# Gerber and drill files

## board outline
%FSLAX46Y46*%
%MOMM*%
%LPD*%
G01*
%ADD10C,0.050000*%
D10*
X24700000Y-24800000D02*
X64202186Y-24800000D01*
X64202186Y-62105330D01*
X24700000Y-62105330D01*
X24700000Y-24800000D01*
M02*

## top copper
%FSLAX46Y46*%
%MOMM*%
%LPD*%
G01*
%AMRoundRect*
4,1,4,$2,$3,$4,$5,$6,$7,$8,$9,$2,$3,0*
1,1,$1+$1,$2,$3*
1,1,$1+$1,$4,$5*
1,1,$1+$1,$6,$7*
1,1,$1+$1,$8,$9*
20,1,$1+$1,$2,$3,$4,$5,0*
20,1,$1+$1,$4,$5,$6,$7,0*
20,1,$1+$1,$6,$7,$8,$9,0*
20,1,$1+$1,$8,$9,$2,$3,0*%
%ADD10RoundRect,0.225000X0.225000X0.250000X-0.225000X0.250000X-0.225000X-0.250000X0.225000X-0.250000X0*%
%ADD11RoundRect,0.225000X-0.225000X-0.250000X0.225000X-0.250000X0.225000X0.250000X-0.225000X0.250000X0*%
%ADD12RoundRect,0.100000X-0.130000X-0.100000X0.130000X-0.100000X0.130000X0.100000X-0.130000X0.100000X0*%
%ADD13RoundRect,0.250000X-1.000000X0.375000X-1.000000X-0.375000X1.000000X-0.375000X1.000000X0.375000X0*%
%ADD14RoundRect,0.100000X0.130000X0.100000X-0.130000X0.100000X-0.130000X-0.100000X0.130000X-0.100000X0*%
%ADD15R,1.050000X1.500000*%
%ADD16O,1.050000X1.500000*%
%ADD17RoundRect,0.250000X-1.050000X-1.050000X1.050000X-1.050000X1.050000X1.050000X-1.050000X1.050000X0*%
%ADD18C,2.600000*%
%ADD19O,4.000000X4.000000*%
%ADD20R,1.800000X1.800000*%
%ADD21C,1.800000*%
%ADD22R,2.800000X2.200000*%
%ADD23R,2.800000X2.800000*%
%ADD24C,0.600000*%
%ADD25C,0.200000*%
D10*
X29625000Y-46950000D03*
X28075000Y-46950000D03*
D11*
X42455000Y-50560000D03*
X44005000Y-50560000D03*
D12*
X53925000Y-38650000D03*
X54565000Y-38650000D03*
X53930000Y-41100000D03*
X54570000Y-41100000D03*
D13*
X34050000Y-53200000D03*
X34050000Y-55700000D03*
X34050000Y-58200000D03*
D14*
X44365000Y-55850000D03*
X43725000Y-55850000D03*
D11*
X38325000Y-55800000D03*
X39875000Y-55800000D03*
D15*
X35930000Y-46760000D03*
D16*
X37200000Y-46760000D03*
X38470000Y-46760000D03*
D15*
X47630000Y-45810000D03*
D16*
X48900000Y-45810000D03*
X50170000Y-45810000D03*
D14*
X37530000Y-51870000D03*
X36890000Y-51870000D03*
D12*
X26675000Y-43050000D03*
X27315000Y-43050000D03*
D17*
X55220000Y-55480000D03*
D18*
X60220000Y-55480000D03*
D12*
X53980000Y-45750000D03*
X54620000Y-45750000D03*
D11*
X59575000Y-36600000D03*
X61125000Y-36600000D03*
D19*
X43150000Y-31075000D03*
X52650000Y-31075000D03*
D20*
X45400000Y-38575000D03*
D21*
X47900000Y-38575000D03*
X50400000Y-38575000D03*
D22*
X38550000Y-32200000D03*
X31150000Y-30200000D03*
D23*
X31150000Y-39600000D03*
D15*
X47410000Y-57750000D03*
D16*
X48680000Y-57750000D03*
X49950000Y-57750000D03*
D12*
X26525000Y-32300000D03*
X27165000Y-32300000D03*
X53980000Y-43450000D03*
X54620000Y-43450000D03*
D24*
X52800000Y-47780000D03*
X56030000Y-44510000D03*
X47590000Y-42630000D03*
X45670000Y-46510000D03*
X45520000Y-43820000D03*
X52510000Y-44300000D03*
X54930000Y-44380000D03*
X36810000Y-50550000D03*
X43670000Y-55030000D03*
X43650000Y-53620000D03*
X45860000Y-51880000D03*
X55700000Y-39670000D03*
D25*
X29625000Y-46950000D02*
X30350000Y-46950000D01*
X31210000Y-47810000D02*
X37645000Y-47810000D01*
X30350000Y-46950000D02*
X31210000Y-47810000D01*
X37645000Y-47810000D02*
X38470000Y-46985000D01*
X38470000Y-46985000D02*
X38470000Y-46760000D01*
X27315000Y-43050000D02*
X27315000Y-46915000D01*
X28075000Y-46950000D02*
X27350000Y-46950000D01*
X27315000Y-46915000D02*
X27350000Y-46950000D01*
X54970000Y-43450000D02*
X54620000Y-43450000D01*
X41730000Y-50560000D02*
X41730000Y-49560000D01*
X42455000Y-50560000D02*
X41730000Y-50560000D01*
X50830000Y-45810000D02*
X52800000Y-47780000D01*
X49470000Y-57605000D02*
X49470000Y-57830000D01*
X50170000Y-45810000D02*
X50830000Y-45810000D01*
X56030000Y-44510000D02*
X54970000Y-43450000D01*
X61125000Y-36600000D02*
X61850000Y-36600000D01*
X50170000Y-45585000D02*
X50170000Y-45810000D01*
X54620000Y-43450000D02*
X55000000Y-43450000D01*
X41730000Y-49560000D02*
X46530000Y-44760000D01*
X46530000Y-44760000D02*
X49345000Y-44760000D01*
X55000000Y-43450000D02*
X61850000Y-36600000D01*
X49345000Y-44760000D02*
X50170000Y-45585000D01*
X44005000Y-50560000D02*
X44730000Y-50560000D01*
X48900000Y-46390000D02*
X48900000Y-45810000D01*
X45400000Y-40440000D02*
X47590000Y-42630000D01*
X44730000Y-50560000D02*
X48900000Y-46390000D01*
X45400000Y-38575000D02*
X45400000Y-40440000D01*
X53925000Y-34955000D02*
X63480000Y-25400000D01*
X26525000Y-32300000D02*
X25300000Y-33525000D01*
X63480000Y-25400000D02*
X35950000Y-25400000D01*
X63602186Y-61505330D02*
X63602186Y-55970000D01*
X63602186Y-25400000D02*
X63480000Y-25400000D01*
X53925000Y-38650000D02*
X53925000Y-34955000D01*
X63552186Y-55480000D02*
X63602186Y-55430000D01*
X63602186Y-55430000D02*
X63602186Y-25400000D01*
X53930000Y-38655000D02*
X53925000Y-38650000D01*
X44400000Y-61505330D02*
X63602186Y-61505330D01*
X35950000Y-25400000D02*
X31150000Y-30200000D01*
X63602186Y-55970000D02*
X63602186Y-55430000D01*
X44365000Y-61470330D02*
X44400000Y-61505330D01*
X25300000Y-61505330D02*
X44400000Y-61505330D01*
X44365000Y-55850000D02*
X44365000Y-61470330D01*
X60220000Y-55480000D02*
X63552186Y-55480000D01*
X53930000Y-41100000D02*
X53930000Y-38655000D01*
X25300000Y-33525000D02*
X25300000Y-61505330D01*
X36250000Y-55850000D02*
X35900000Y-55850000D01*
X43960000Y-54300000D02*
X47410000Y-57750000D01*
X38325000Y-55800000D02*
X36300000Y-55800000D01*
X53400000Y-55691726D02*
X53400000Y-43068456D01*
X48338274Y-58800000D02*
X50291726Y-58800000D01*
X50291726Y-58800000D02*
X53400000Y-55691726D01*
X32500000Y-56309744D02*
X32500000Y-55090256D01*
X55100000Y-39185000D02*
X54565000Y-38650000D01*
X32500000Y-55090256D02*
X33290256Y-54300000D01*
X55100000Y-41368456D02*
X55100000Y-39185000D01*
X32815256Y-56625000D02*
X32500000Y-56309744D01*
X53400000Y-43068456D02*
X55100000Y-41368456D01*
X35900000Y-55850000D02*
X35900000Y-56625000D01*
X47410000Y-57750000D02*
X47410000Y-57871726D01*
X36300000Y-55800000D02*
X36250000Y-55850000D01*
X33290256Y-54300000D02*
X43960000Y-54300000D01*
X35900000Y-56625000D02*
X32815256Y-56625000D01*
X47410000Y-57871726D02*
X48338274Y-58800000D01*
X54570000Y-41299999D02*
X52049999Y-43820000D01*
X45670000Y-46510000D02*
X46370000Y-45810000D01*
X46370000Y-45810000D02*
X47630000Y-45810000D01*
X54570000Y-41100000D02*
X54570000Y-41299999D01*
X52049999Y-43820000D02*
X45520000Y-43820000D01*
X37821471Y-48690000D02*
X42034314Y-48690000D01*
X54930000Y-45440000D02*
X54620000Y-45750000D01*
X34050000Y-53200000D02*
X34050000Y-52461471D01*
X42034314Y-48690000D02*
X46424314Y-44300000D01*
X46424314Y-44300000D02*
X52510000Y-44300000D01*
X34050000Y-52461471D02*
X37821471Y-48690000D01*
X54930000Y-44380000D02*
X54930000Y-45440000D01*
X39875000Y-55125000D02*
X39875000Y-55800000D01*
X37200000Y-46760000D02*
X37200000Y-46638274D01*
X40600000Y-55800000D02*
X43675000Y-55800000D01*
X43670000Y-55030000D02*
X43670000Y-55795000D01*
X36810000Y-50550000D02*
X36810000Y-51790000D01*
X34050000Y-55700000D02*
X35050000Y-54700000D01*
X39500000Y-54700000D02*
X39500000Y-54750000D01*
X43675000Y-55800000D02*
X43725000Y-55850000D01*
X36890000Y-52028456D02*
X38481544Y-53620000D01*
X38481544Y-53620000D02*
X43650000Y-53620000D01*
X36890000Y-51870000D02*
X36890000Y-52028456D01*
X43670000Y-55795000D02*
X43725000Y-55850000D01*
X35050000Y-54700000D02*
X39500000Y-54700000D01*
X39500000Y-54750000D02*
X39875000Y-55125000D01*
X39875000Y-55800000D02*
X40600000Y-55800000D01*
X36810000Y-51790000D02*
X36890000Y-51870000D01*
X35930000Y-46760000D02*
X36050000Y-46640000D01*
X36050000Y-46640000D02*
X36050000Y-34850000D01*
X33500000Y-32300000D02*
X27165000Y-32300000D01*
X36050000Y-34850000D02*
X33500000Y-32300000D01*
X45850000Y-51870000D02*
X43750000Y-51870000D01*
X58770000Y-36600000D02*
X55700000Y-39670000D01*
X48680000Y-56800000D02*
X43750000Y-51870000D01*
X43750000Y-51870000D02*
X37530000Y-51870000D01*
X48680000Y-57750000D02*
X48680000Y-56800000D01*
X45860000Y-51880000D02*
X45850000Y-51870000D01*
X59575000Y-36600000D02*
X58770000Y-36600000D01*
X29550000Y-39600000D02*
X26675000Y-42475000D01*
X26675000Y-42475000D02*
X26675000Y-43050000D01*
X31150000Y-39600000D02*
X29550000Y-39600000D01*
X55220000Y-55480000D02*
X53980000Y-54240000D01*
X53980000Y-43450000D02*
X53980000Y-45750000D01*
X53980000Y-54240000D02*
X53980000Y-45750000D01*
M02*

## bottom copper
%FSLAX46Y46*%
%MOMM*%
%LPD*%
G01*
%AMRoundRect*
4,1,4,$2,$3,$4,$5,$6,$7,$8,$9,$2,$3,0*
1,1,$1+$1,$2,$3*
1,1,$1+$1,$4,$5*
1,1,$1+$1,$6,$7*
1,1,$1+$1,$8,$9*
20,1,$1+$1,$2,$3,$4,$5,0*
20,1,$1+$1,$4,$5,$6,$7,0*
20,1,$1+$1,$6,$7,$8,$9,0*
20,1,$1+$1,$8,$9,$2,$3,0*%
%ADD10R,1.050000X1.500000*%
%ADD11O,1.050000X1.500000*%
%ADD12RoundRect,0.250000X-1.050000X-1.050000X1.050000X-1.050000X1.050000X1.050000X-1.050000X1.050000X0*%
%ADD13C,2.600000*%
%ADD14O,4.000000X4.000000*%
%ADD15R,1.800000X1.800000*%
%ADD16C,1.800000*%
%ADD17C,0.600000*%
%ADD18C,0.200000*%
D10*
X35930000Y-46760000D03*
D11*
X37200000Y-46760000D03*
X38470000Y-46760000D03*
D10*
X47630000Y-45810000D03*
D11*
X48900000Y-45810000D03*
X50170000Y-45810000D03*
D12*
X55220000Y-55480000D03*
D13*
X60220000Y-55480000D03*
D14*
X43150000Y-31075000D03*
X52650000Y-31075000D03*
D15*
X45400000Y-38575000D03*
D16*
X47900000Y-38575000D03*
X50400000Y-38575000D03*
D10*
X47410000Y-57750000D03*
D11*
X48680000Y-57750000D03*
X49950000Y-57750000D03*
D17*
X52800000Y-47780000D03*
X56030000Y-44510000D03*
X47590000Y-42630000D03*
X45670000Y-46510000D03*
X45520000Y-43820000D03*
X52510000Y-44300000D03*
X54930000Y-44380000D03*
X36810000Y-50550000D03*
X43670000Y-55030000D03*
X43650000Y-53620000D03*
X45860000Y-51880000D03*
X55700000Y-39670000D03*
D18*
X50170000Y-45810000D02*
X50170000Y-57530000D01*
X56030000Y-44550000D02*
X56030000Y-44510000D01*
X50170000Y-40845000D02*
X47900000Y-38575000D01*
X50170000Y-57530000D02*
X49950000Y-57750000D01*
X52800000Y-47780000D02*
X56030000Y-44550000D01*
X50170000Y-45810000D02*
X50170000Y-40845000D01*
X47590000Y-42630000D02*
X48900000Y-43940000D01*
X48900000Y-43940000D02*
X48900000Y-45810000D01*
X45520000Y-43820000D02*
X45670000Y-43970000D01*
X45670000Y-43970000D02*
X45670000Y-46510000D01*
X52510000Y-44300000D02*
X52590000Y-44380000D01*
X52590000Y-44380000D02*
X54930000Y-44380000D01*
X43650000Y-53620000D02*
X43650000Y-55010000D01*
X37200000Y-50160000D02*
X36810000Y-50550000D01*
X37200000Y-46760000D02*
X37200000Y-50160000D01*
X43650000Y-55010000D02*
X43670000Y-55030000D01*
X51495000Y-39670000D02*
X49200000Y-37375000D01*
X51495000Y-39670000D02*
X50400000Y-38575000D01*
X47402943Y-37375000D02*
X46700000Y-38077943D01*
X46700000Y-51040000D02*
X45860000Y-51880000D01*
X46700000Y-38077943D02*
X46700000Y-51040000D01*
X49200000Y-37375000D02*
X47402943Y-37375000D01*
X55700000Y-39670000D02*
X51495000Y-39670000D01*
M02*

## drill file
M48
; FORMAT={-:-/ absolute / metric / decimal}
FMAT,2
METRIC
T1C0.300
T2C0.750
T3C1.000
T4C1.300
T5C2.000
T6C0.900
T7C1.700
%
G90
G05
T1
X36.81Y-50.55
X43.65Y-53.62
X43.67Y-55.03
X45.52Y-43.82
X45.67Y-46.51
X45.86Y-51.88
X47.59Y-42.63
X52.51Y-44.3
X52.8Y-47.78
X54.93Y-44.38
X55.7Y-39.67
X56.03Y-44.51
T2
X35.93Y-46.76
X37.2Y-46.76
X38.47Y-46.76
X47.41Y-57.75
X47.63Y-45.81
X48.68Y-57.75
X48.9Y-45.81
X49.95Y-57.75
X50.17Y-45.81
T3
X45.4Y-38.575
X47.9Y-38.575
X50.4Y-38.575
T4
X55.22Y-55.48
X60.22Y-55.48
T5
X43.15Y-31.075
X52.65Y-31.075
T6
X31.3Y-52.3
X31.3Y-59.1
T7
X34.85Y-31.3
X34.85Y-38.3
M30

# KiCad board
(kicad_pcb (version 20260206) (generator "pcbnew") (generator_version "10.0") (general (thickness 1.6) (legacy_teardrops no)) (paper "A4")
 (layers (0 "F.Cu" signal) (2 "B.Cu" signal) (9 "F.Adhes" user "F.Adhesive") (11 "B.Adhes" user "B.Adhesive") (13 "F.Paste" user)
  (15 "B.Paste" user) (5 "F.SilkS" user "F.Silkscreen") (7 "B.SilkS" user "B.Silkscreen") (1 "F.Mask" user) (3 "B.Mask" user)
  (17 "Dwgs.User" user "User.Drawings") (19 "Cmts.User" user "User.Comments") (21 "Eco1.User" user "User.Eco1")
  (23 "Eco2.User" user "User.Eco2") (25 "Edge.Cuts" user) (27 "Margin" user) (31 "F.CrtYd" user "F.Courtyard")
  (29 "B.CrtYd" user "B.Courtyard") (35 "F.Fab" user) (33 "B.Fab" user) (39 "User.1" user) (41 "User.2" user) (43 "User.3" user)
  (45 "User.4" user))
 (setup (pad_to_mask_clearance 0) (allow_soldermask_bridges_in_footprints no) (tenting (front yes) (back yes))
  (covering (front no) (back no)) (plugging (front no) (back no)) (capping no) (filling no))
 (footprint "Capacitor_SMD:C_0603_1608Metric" (layer "F.Cu") (at 28.85 46.95 180)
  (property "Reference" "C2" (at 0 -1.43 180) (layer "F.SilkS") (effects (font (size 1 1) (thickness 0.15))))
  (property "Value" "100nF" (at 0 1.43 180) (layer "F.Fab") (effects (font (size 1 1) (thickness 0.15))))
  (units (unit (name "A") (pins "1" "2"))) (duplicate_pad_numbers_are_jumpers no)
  (pad "1" smd roundrect (at -0.775 0 180) (size 0.9 0.95) (layers "F.Cu" "F.Mask" "F.Paste") (roundrect_rratio 0.25) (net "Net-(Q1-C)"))
  (pad "2" smd roundrect (at 0.775 0 180) (size 0.9 0.95) (layers "F.Cu" "F.Mask" "F.Paste") (roundrect_rratio 0.25) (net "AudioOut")))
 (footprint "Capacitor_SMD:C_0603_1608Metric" (layer "F.Cu") (at 43.23 50.56)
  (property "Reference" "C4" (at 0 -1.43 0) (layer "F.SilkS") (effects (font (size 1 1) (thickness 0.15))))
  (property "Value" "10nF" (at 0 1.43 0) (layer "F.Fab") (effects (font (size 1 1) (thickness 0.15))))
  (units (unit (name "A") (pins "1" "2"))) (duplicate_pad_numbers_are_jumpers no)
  (pad "1" smd roundrect (at -0.775 0) (size 0.9 0.95) (layers "F.Cu" "F.Mask" "F.Paste") (roundrect_rratio 0.25) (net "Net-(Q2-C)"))
  (pad "2" smd roundrect (at 0.775 0) (size 0.9 0.95) (layers "F.Cu" "F.Mask" "F.Paste") (roundrect_rratio 0.25) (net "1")))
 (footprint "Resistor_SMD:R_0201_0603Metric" (layer "F.Cu") (at 54.245 38.65)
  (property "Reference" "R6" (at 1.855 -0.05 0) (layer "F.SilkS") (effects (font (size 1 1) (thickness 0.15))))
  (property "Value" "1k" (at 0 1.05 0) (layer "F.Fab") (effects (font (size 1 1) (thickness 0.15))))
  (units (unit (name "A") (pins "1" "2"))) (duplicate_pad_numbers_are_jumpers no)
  (pad "" smd roundrect (at -0.345 0) (size 0.318 0.36) (layers "F.Paste") (roundrect_rratio 0.25))
  (pad "" smd roundrect (at 0.345 0) (size 0.318 0.36) (layers "F.Paste") (roundrect_rratio 0.25))
  (pad "1" smd roundrect (at -0.32 0) (size 0.46 0.4) (layers "F.Cu" "F.Mask") (roundrect_rratio 0.25) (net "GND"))
  (pad "2" smd roundrect (at 0.32 0) (size 0.46 0.4) (layers "F.Cu" "F.Mask") (roundrect_rratio 0.25) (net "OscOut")))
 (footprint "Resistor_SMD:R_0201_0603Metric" (layer "F.Cu") (at 54.25 41.1)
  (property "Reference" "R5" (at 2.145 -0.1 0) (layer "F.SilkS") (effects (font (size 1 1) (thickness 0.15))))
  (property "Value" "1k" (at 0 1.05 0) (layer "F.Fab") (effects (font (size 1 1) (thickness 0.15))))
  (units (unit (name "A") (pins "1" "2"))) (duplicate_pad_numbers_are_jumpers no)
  (pad "" smd roundrect (at -0.345 0) (size 0.318 0.36) (layers "F.Paste") (roundrect_rratio 0.25))
  (pad "" smd roundrect (at 0.345 0) (size 0.318 0.36) (layers "F.Paste") (roundrect_rratio 0.25))
  (pad "1" smd roundrect (at -0.32 0) (size 0.46 0.4) (layers "F.Cu" "F.Mask") (roundrect_rratio 0.25) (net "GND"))
  (pad "2" smd roundrect (at 0.32 0) (size 0.46 0.4) (layers "F.Cu" "F.Mask") (roundrect_rratio 0.25) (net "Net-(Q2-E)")))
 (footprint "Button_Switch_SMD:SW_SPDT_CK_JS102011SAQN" (layer "F.Cu") (at 31.3 55.7 -90)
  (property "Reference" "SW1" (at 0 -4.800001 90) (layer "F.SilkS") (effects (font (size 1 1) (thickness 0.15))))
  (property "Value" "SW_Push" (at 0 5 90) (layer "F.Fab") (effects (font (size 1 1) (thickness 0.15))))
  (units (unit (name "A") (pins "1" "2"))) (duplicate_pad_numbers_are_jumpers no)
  (pad "" np_thru_hole circle (at -3.4 0 270) (size 0.9 0.9) (drill 0.9) (layers "*.Cu" "*.Mask"))
  (pad "" np_thru_hole circle (at 3.4 0 270) (size 0.9 0.9) (drill 0.9) (layers "*.Cu" "*.Mask"))
  (pad "1" smd roundrect (at -2.5 -2.75 270) (size 1.25 2.5) (layers "F.Cu" "F.Mask" "F.Paste") (roundrect_rratio 0.2) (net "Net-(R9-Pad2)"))
  (pad "2" smd roundrect (at 0 -2.75 270) (size 1.25 2.5) (layers "F.Cu" "F.Mask" "F.Paste") (roundrect_rratio 0.2) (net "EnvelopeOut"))
  (pad "3" smd roundrect (at 2.5 -2.75 270) (size 1.25 2.5) (layers "F.Cu" "F.Mask" "F.Paste") (roundrect_rratio 0.2)))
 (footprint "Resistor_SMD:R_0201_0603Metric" (layer "F.Cu") (at 44.045 55.85 180)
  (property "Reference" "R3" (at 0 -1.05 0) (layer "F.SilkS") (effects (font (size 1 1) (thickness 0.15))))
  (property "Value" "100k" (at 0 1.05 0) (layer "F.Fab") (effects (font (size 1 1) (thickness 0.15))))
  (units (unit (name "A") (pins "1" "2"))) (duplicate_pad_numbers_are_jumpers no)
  (pad "" smd roundrect (at -0.345 0 180) (size 0.318 0.36) (layers "F.Paste") (roundrect_rratio 0.25))
  (pad "" smd roundrect (at 0.345 0 180) (size 0.318 0.36) (layers "F.Paste") (roundrect_rratio 0.25))
  (pad "1" smd roundrect (at -0.32 0 180) (size 0.46 0.4) (layers "F.Cu" "F.Mask") (roundrect_rratio 0.25) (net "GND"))
  (pad "2" smd roundrect (at 0.32 0 180) (size 0.46 0.4) (layers "F.Cu" "F.Mask") (roundrect_rratio 0.25) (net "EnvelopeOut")))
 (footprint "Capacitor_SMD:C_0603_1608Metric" (layer "F.Cu") (at 39.1 55.8)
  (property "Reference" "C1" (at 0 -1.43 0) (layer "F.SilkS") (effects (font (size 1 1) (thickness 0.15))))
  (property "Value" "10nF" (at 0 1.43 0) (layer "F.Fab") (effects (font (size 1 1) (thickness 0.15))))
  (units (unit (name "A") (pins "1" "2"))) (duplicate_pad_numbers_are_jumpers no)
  (pad "1" smd roundrect (at -0.775 0) (size 0.9 0.95) (layers "F.Cu" "F.Mask" "F.Paste") (roundrect_rratio 0.25) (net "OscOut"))
  (pad "2" smd roundrect (at 0.775 0) (size 0.9 0.95) (layers "F.Cu" "F.Mask" "F.Paste") (roundrect_rratio 0.25) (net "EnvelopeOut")))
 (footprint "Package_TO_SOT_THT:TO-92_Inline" (layer "F.Cu") (at 35.93 46.76)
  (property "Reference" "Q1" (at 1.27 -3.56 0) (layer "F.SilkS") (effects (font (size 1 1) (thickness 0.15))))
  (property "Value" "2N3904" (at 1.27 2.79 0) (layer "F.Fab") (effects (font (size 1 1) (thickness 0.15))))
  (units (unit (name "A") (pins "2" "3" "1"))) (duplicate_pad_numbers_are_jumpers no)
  (pad "1" thru_hole rect (at 0 0) (size 1.05 1.5) (drill 0.75) (layers "*.Cu" "*.Mask") (remove_unused_layers no) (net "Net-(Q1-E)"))
  (pad "2" thru_hole oval (at 1.27 0) (size 1.05 1.5) (drill 0.75) (layers "*.Cu" "*.Mask") (remove_unused_layers no) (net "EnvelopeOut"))
  (pad "3" thru_hole oval (at 2.54 0) (size 1.05 1.5) (drill 0.75) (layers "*.Cu" "*.Mask") (remove_unused_layers no) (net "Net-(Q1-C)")))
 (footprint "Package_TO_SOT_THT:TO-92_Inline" (layer "F.Cu") (at 47.63 45.81)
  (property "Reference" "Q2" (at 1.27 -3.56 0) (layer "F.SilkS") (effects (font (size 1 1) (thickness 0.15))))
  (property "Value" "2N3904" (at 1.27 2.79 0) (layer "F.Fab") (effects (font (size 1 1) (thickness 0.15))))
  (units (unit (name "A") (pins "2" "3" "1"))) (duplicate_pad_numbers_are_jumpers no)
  (pad "1" thru_hole rect (at 0 0) (size 1.05 1.5) (drill 0.75) (layers "*.Cu" "*.Mask") (remove_unused_layers no) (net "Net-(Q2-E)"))
  (pad "2" thru_hole oval (at 1.27 0) (size 1.05 1.5) (drill 0.75) (layers "*.Cu" "*.Mask") (remove_unused_layers no) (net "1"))
  (pad "3" thru_hole oval (at 2.54 0) (size 1.05 1.5) (drill 0.75) (layers "*.Cu" "*.Mask") (remove_unused_layers no) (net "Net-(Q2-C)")))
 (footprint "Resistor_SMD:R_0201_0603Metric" (layer "F.Cu") (at 37.21 51.87 180)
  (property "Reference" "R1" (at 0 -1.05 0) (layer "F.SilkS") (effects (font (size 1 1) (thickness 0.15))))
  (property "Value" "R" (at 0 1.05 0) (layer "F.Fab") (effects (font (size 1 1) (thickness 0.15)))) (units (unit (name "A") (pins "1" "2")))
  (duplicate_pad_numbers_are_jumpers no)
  (pad "" smd roundrect (at -0.345 0 180) (size 0.318 0.36) (layers "F.Paste") (roundrect_rratio 0.25))
  (pad "" smd roundrect (at 0.345 0 180) (size 0.318 0.36) (layers "F.Paste") (roundrect_rratio 0.25))
  (pad "1" smd roundrect (at -0.32 0 180) (size 0.46 0.4) (layers "F.Cu" "F.Mask") (roundrect_rratio 0.25) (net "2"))
  (pad "2" smd roundrect (at 0.32 0 180) (size 0.46 0.4) (layers "F.Cu" "F.Mask") (roundrect_rratio 0.25) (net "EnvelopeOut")))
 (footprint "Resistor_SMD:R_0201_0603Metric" (layer "F.Cu") (at 26.995 43.05)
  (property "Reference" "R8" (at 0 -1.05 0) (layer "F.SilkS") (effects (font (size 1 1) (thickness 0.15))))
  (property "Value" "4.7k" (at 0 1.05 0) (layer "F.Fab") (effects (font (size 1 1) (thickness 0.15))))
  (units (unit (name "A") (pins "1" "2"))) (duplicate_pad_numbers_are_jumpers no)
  (pad "" smd roundrect (at -0.345 0) (size 0.318 0.36) (layers "F.Paste") (roundrect_rratio 0.25))
  (pad "" smd roundrect (at 0.345 0) (size 0.318 0.36) (layers "F.Paste") (roundrect_rratio 0.25))
  (pad "1" smd roundrect (at -0.32 0) (size 0.46 0.4) (layers "F.Cu" "F.Mask") (roundrect_rratio 0.25) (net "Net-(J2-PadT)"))
  (pad "2" smd roundrect (at 0.32 0) (size 0.46 0.4) (layers "F.Cu" "F.Mask") (roundrect_rratio 0.25) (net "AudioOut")))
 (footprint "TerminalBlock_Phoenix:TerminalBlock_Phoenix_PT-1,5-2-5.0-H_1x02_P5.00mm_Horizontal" (layer "F.Cu") (at 55.22 55.48)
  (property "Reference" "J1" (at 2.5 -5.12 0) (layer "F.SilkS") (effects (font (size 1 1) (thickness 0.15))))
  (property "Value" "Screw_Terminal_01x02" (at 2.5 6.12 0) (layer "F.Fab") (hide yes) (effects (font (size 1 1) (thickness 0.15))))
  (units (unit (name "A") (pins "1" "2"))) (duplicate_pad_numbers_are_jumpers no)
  (pad "1" thru_hole roundrect (at 0 0) (size 2.6 2.6) (drill 1.3) (layers "*.Cu" "*.Mask") (remove_unused_layers no)
   (roundrect_rratio 0.096154) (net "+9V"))
  (pad "2" thru_hole circle (at 5 0) (size 2.6 2.6) (drill 1.3) (layers "*.Cu" "*.Mask") (remove_unused_layers no) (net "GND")))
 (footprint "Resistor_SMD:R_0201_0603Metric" (layer "F.Cu") (at 54.3 45.75)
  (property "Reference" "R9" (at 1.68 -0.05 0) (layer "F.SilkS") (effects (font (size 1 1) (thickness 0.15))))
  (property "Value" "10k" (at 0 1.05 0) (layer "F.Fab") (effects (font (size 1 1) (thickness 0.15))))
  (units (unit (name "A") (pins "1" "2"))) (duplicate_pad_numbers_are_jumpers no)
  (pad "" smd roundrect (at -0.345 0) (size 0.318 0.36) (layers "F.Paste") (roundrect_rratio 0.25))
  (pad "" smd roundrect (at 0.345 0) (size 0.318 0.36) (layers "F.Paste") (roundrect_rratio 0.25))
  (pad "1" smd roundrect (at -0.32 0) (size 0.46 0.4) (layers "F.Cu" "F.Mask") (roundrect_rratio 0.25) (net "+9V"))
  (pad "2" smd roundrect (at 0.32 0) (size 0.46 0.4) (layers "F.Cu" "F.Mask") (roundrect_rratio 0.25) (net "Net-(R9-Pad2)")))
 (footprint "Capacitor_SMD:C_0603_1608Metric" (layer "F.Cu") (at 60.35 36.6)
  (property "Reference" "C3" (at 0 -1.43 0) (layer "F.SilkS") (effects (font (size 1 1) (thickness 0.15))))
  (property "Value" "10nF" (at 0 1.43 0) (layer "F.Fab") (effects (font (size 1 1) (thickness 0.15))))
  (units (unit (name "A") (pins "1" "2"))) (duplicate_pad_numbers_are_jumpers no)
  (pad "1" smd roundrect (at -0.775 0) (size 0.9 0.95) (layers "F.Cu" "F.Mask" "F.Paste") (roundrect_rratio 0.25) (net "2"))
  (pad "2" smd roundrect (at 0.775 0) (size 0.9 0.95) (layers "F.Cu" "F.Mask" "F.Paste") (roundrect_rratio 0.25) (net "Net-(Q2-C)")))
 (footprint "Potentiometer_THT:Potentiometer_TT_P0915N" (layer "F.Cu") (at 45.4 38.575)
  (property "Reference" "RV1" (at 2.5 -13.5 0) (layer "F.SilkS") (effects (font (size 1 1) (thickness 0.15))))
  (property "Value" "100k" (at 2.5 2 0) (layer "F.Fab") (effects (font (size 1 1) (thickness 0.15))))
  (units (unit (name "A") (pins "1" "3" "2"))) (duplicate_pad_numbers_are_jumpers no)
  (pad "" thru_hole oval (at -2.25 -7.5) (size 4 4) (drill 2) (layers "*.Cu" "*.Mask") (remove_unused_layers no))
  (pad "" thru_hole oval (at 7.25 -7.5) (size 4 4) (drill 2) (layers "*.Cu" "*.Mask") (remove_unused_layers no))
  (pad "1" thru_hole rect (at 0 0) (size 1.8 1.8) (drill 1) (layers "*.Cu" "*.Mask") (remove_unused_layers no) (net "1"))
  (pad "2" thru_hole circle (at 2.5 0) (size 1.8 1.8) (drill 1) (layers "*.Cu" "*.Mask") (remove_unused_layers no) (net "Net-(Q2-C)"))
  (pad "3" thru_hole circle (at 5 0) (size 1.8 1.8) (drill 1) (layers "*.Cu" "*.Mask") (remove_unused_layers no) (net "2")))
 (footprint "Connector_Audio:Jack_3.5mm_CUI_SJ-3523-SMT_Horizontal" (layer "F.Cu") (at 34.85 33.8)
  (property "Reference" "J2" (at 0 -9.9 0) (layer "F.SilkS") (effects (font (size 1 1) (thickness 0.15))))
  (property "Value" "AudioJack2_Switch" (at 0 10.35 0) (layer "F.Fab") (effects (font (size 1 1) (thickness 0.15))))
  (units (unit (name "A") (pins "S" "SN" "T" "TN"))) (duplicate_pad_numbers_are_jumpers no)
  (pad "" np_thru_hole circle (at 0 -2.5) (size 1.7 1.7) (drill 1.7) (layers "*.Cu" "*.Mask"))
  (pad "" np_thru_hole circle (at 0 4.5) (size 1.7 1.7) (drill 1.7) (layers "*.Cu" "*.Mask"))
  (pad "R" smd rect (at 3.7 -1.6) (size 2.8 2.2) (layers "F.Cu" "F.Mask" "F.Paste"))
  (pad "S" smd rect (at -3.7 -3.6) (size 2.8 2.2) (layers "F.Cu" "F.Mask" "F.Paste") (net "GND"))
  (pad "T" smd rect (at -3.7 5.8) (size 2.8 2.8) (layers "F.Cu" "F.Mask" "F.Paste") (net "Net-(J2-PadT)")))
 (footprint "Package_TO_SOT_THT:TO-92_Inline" (layer "F.Cu") (at 47.41 57.75)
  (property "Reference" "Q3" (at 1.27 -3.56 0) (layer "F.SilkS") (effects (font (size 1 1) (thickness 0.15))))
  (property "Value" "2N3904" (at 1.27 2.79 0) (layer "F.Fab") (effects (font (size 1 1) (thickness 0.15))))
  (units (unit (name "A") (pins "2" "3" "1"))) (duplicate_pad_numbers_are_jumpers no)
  (pad "1" thru_hole rect (at 0 0) (size 1.05 1.5) (drill 0.75) (layers "*.Cu" "*.Mask") (remove_unused_layers no) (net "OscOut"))
  (pad "2" thru_hole oval (at 1.27 0) (size 1.05 1.5) (drill 0.75) (layers "*.Cu" "*.Mask") (remove_unused_layers no) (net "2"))
  (pad "3" thru_hole oval (at 2.54 0) (size 1.05 1.5) (drill 0.75) (layers "*.Cu" "*.Mask") (remove_unused_layers no) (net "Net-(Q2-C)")))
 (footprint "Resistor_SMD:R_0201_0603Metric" (layer "F.Cu") (at 26.845 32.3)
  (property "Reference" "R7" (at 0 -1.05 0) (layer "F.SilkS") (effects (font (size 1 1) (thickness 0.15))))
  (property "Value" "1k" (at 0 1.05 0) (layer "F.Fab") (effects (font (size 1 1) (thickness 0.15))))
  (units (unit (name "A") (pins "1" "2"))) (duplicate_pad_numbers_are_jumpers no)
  (pad "" smd roundrect (at -0.345 0) (size 0.318 0.36) (layers "F.Paste") (roundrect_rratio 0.25))
  (pad "" smd roundrect (at 0.345 0) (size 0.318 0.36) (layers "F.Paste") (roundrect_rratio 0.25))
  (pad "1" smd roundrect (at -0.32 0) (size 0.46 0.4) (layers "F.Cu" "F.Mask") (roundrect_rratio 0.25) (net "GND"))
  (pad "2" smd roundrect (at 0.32 0) (size 0.46 0.4) (layers "F.Cu" "F.Mask") (roundrect_rratio 0.25) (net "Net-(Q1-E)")))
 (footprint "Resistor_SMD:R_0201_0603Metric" (layer "F.Cu") (at 54.3 43.45)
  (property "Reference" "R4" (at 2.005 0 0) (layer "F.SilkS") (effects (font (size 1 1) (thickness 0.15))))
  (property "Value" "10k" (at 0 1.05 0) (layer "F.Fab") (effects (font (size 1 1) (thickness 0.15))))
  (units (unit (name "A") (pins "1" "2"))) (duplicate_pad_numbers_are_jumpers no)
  (pad "" smd roundrect (at -0.345 0) (size 0.318 0.36) (layers "F.Paste") (roundrect_rratio 0.25))
  (pad "" smd roundrect (at 0.345 0) (size 0.318 0.36) (layers "F.Paste") (roundrect_rratio 0.25))
  (pad "1" smd roundrect (at -0.32 0) (size 0.46 0.4) (layers "F.Cu" "F.Mask") (roundrect_rratio 0.25) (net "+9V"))
  (pad "2" smd roundrect (at 0.32 0) (size 0.46 0.4) (layers "F.Cu" "F.Mask") (roundrect_rratio 0.25) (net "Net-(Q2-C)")))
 (gr_rect (start 24.7 24.8) (end 64.202186 62.10533) (stroke (width 0.05) (type default)) (fill no) (layer "Edge.Cuts"))
 (segment (start 29.625 46.95) (end 30.35 46.95) (width 0.2) (layer "F.Cu") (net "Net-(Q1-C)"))
 (segment (start 31.21 47.81) (end 37.645 47.81) (width 0.2) (layer "F.Cu") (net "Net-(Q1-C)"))
 (segment (start 30.35 46.95) (end 31.21 47.81) (width 0.2) (layer "F.Cu") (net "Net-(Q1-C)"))
 (segment (start 37.645 47.81) (end 38.47 46.985) (width 0.2) (layer "F.Cu") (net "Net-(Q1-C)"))
 (segment (start 38.47 46.985) (end 38.47 46.76) (width 0.2) (layer "F.Cu") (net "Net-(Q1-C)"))
 (segment (start 27.315 43.05) (end 27.315 46.915) (width 0.2) (layer "F.Cu") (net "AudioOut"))
 (segment (start 28.075 46.95) (end 27.35 46.95) (width 0.2) (layer "F.Cu") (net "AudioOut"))
 (segment (start 27.315 46.915) (end 27.35 46.95) (width 0.2) (layer "F.Cu") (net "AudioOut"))
 (segment (start 54.97 43.45) (end 54.62 43.45) (width 0.2) (layer "F.Cu") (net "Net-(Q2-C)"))
 (segment (start 41.73 50.56) (end 41.73 49.56) (width 0.2) (layer "F.Cu") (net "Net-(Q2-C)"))
 (segment (start 42.455 50.56) (end 41.73 50.56) (width 0.2) (layer "F.Cu") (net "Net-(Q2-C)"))
 (segment (start 50.83 45.81) (end 52.8 47.78) (width 0.2) (layer "F.Cu") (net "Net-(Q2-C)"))
 (segment (start 49.47 57.605) (end 49.47 57.83) (width 0.2) (layer "F.Cu") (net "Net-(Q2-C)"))
 (segment (start 50.17 45.81) (end 50.83 45.81) (width 0.2) (layer "F.Cu") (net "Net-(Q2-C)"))
 (segment (start 56.03 44.51) (end 54.97 43.45) (width 0.2) (layer "F.Cu") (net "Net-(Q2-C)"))
 (segment (start 61.125 36.6) (end 61.85 36.6) (width 0.2) (layer "F.Cu") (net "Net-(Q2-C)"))
 (segment (start 50.17 45.585) (end 50.17 45.81) (width 0.2) (layer "F.Cu") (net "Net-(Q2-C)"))
 (segment (start 54.62 43.45) (end 55 43.45) (width 0.2) (layer "F.Cu") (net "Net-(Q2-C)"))
 (segment (start 41.73 49.56) (end 46.53 44.76) (width 0.2) (layer "F.Cu") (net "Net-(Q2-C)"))
 (segment (start 46.53 44.76) (end 49.345 44.76) (width 0.2) (layer "F.Cu") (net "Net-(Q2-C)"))
 (segment (start 55 43.45) (end 61.85 36.6) (width 0.2) (layer "F.Cu") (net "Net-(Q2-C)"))
 (segment (start 49.345 44.76) (end 50.17 45.585) (width 0.2) (layer "F.Cu") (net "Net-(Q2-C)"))
 (via (at 52.8 47.78) (size 0.6) (drill 0.3) (layers "F.Cu" "B.Cu") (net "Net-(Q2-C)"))
 (via (at 56.03 44.51) (size 0.6) (drill 0.3) (layers "F.Cu" "B.Cu") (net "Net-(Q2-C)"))
 (segment (start 50.17 45.81) (end 50.17 57.53) (width 0.2) (layer "B.Cu") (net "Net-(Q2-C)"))
 (segment (start 56.03 44.55) (end 56.03 44.51) (width 0.2) (layer "B.Cu") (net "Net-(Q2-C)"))
 (segment (start 50.17 40.845) (end 47.9 38.575) (width 0.2) (layer "B.Cu") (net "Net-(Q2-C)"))
 (segment (start 50.17 57.53) (end 49.95 57.75) (width 0.2) (layer "B.Cu") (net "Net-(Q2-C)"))
 (segment (start 52.8 47.78) (end 56.03 44.55) (width 0.2) (layer "B.Cu") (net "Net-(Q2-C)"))
 (segment (start 50.17 45.81) (end 50.17 40.845) (width 0.2) (layer "B.Cu") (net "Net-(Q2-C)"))
 (segment (start 44.005 50.56) (end 44.73 50.56) (width 0.2) (layer "F.Cu") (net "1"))
 (segment (start 48.9 46.39) (end 48.9 45.81) (width 0.2) (layer "F.Cu") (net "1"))
 (segment (start 45.4 40.44) (end 47.59 42.63) (width 0.2) (layer "F.Cu") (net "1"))
 (segment (start 44.73 50.56) (end 48.9 46.39) (width 0.2) (layer "F.Cu") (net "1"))
 (segment (start 45.4 38.575) (end 45.4 40.44) (width 0.2) (layer "F.Cu") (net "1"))
 (via (at 47.59 42.63) (size 0.6) (drill 0.3) (layers "F.Cu" "B.Cu") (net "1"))
 (segment (start 47.59 42.63) (end 48.9 43.94) (width 0.2) (layer "B.Cu") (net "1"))
 (segment (start 48.9 43.94) (end 48.9 45.81) (width 0.2) (layer "B.Cu") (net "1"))
 (segment (start 53.925 34.955) (end 63.48 25.4) (width 0.2) (layer "F.Cu") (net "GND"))
 (segment (start 26.525 32.3) (end 25.3 33.525) (width 0.2) (layer "F.Cu") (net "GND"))
 (segment (start 63.48 25.4) (end 35.95 25.4) (width 0.2) (layer "F.Cu") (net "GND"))
 (segment (start 63.602186 61.50533) (end 63.602186 55.97) (width 0.2) (layer "F.Cu") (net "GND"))
 (segment (start 63.602186 25.4) (end 63.48 25.4) (width 0.2) (layer "F.Cu") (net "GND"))
 (segment (start 53.925 38.65) (end 53.925 34.955) (width 0.2) (layer "F.Cu") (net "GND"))
 (segment (start 63.552186 55.48) (end 63.602186 55.43) (width 0.2) (layer "F.Cu") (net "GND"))
 (segment (start 63.602186 55.43) (end 63.602186 25.4) (width 0.2) (layer "F.Cu") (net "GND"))
 (segment (start 53.93 38.655) (end 53.925 38.65) (width 0.2) (layer "F.Cu") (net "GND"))
 (segment (start 44.4 61.50533) (end 63.602186 61.50533) (width 0.2) (layer "F.Cu") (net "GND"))
 (segment (start 35.95 25.4) (end 31.15 30.2) (width 0.2) (layer "F.Cu") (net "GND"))
 (segment (start 63.602186 55.97) (end 63.602186 55.43) (width 0.2) (layer "F.Cu") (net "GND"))
 (segment (start 44.365 61.47033) (end 44.4 61.50533) (width 0.2) (layer "F.Cu") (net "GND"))
 (segment (start 25.3 61.50533) (end 44.4 61.50533) (width 0.2) (layer "F.Cu") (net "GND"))
 (segment (start 44.365 55.85) (end 44.365 61.47033) (width 0.2) (layer "F.Cu") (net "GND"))
 (segment (start 60.22 55.48) (end 63.552186 55.48) (width 0.2) (layer "F.Cu") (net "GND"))
 (segment (start 53.93 41.1) (end 53.93 38.655) (width 0.2) (layer "F.Cu") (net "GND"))
 (segment (start 25.3 33.525) (end 25.3 61.50533) (width 0.2) (layer "F.Cu") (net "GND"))
 (segment (start 36.25 55.85) (end 35.9 55.85) (width 0.2) (layer "F.Cu") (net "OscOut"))
 (segment (start 43.96 54.3) (end 47.41 57.75) (width 0.2) (layer "F.Cu") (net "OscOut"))
 (segment (start 38.325 55.8) (end 36.3 55.8) (width 0.2) (layer "F.Cu") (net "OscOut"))
 (segment (start 53.4 55.691726) (end 53.4 43.068456) (width 0.2) (layer "F.Cu") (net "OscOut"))
 (segment (start 48.338274 58.8) (end 50.291726 58.8) (width 0.2) (layer "F.Cu") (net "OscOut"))
 (segment (start 50.291726 58.8) (end 53.4 55.691726) (width 0.2) (layer "F.Cu") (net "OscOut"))
 (segment (start 32.5 56.309744) (end 32.5 55.090256) (width 0.2) (layer "F.Cu") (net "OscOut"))
 (segment (start 55.1 39.185) (end 54.565 38.65) (width 0.2) (layer "F.Cu") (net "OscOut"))
 (segment (start 32.5 55.090256) (end 33.290256 54.3) (width 0.2) (layer "F.Cu") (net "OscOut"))
 (segment (start 55.1 41.368456) (end 55.1 39.185) (width 0.2) (layer "F.Cu") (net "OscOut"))
 (segment (start 32.815256 56.625) (end 32.5 56.309744) (width 0.2) (layer "F.Cu") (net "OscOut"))
 (segment (start 53.4 43.068456) (end 55.1 41.368456) (width 0.2) (layer "F.Cu") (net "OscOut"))
 (segment (start 35.9 55.85) (end 35.9 56.625) (width 0.2) (layer "F.Cu") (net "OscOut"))
 (segment (start 47.41 57.75) (end 47.41 57.871726) (width 0.2) (layer "F.Cu") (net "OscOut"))
 (segment (start 36.3 55.8) (end 36.25 55.85) (width 0.2) (layer "F.Cu") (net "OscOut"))
 (segment (start 33.290256 54.3) (end 43.96 54.3) (width 0.2) (layer "F.Cu") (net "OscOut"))
 (segment (start 35.9 56.625) (end 32.815256 56.625) (width 0.2) (layer "F.Cu") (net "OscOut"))
 (segment (start 47.41 57.871726) (end 48.338274 58.8) (width 0.2) (layer "F.Cu") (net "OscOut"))
 (segment (start 54.57 41.299999) (end 52.049999 43.82) (width 0.2) (layer "F.Cu") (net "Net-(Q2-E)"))
 (segment (start 45.67 46.51) (end 46.37 45.81) (width 0.2) (layer "F.Cu") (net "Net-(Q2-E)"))
 (segment (start 46.37 45.81) (end 47.63 45.81) (width 0.2) (layer "F.Cu") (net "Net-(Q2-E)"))
 (segment (start 54.57 41.1) (end 54.57 41.299999) (width 0.2) (layer "F.Cu") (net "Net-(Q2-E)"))
 (segment (start 52.049999 43.82) (end 45.52 43.82) (width 0.2) (layer "F.Cu") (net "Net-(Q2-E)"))
 (via (at 45.67 46.51) (size 0.6) (drill 0.3) (layers "F.Cu" "B.Cu") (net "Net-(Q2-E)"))
 (via (at 45.52 43.82) (size 0.6) (drill 0.3) (layers "F.Cu" "B.Cu") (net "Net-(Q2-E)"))
 (segment (start 45.52 43.82) (end 45.67 43.97) (width 0.2) (layer "B.Cu") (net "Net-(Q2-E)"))
 (segment (start 45.67 43.97) (end 45.67 46.51) (width 0.2) (layer "B.Cu") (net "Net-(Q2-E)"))
 (segment (start 37.821471 48.69) (end 42.034314 48.69) (width 0.2) (layer "F.Cu") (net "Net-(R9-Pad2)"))
 (segment (start 54.93 45.44) (end 54.62 45.75) (width 0.2) (layer "F.Cu") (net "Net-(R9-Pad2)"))
 (segment (start 34.05 53.2) (end 34.05 52.461471) (width 0.2) (layer "F.Cu") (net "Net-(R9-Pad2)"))
 (segment (start 42.034314 48.69) (end 46.424314 44.3) (width 0.2) (layer "F.Cu") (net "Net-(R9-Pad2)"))
 (segment (start 46.424314 44.3) (end 52.51 44.3) (width 0.2) (layer "F.Cu") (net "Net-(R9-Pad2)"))
 (segment (start 34.05 52.461471) (end 37.821471 48.69) (width 0.2) (layer "F.Cu") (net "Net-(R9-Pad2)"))
 (segment (start 54.93 44.38) (end 54.93 45.44) (width 0.2) (layer "F.Cu") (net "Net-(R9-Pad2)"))
 (via (at 52.51 44.3) (size 0.6) (drill 0.3) (layers "F.Cu" "B.Cu") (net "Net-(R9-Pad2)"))
 (via (at 54.93 44.38) (size 0.6) (drill 0.3) (layers "F.Cu" "B.Cu") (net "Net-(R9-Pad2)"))
 (segment (start 52.51 44.3) (end 52.59 44.38) (width 0.2) (layer "B.Cu") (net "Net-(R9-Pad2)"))
 (segment (start 52.59 44.38) (end 54.93 44.38) (width 0.2) (layer "B.Cu") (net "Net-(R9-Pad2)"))
 (segment (start 39.875 55.125) (end 39.875 55.8) (width 0.2) (layer "F.Cu") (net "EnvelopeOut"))
 (segment (start 37.2 46.76) (end 37.2 46.638274) (width 0.2) (layer "F.Cu") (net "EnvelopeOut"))
 (segment (start 40.6 55.8) (end 43.675 55.8) (width 0.2) (layer "F.Cu") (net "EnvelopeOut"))
 (segment (start 43.67 55.03) (end 43.67 55.795) (width 0.2) (layer "F.Cu") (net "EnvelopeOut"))
 (segment (start 36.81 50.55) (end 36.81 51.79) (width 0.2) (layer "F.Cu") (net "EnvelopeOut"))
 (segment (start 34.05 55.7) (end 35.05 54.7) (width 0.2) (layer "F.Cu") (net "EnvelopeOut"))
 (segment (start 39.5 54.7) (end 39.5 54.75) (width 0.2) (layer "F.Cu") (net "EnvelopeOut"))
 (segment (start 43.675 55.8) (end 43.725 55.85) (width 0.2) (layer "F.Cu") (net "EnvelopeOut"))
 (segment (start 36.89 52.028456) (end 38.481544 53.62) (width 0.2) (layer "F.Cu") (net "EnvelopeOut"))
 (segment (start 38.481544 53.62) (end 43.65 53.62) (width 0.2) (layer "F.Cu") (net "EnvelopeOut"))
 (segment (start 36.89 51.87) (end 36.89 52.028456) (width 0.2) (layer "F.Cu") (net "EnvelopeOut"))
 (segment (start 43.67 55.795) (end 43.725 55.85) (width 0.2) (layer "F.Cu") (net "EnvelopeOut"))
 (segment (start 35.05 54.7) (end 39.5 54.7) (width 0.2) (layer "F.Cu") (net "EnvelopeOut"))
 (segment (start 39.5 54.75) (end 39.875 55.125) (width 0.2) (layer "F.Cu") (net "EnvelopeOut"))
 (segment (start 39.875 55.8) (end 40.6 55.8) (width 0.2) (layer "F.Cu") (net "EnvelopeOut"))
 (segment (start 36.81 51.79) (end 36.89 51.87) (width 0.2) (layer "F.Cu") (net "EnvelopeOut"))
 (via (at 36.81 50.55) (size 0.6) (drill 0.3) (layers "F.Cu" "B.Cu") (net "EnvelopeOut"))
 (via (at 43.67 55.03) (size 0.6) (drill 0.3) (layers "F.Cu" "B.Cu") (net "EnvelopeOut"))
 (via (at 43.65 53.62) (size 0.6) (drill 0.3) (layers "F.Cu" "B.Cu") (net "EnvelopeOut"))
 (segment (start 43.65 53.62) (end 43.65 55.01) (width 0.2) (layer "B.Cu") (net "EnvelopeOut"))
 (segment (start 37.2 50.16) (end 36.81 50.55) (width 0.2) (layer "B.Cu") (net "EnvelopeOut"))
 (segment (start 37.2 46.76) (end 37.2 50.16) (width 0.2) (layer "B.Cu") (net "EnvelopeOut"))
 (segment (start 43.65 55.01) (end 43.67 55.03) (width 0.2) (layer "B.Cu") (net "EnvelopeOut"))
 (segment (start 35.93 46.76) (end 36.05 46.64) (width 0.2) (layer "F.Cu") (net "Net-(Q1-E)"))
 (segment (start 36.05 46.64) (end 36.05 34.85) (width 0.2) (layer "F.Cu") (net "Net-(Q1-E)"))
 (segment (start 33.5 32.3) (end 27.165 32.3) (width 0.2) (layer "F.Cu") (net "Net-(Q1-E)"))
 (segment (start 36.05 34.85) (end 33.5 32.3) (width 0.2) (layer "F.Cu") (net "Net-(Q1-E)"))
 (segment (start 45.85 51.87) (end 43.75 51.87) (width 0.2) (layer "F.Cu") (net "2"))
 (segment (start 58.77 36.6) (end 55.7 39.67) (width 0.2) (layer "F.Cu") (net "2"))
 (segment (start 48.68 56.8) (end 43.75 51.87) (width 0.2) (layer "F.Cu") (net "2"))
 (segment (start 43.75 51.87) (end 37.53 51.87) (width 0.2) (layer "F.Cu") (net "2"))
 (segment (start 48.68 57.75) (end 48.68 56.8) (width 0.2) (layer "F.Cu") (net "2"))
 (segment (start 45.86 51.88) (end 45.85 51.87) (width 0.2) (layer "F.Cu") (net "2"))
 (segment (start 59.575 36.6) (end 58.77 36.6) (width 0.2) (layer "F.Cu") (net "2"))
 (via (at 45.86 51.88) (size 0.6) (drill 0.3) (layers "F.Cu" "B.Cu") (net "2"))
 (via (at 55.7 39.67) (size 0.6) (drill 0.3) (layers "F.Cu" "B.Cu") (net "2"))
 (segment (start 51.495 39.67) (end 49.2 37.375) (width 0.2) (layer "B.Cu") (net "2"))
 (segment (start 51.495 39.67) (end 50.4 38.575) (width 0.2) (layer "B.Cu") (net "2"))
 (segment (start 47.402943 37.375) (end 46.7 38.077943) (width 0.2) (layer "B.Cu") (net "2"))
 (segment (start 46.7 51.04) (end 45.86 51.88) (width 0.2) (layer "B.Cu") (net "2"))
 (segment (start 46.7 38.077943) (end 46.7 51.04) (width 0.2) (layer "B.Cu") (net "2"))
 (segment (start 49.2 37.375) (end 47.402943 37.375) (width 0.2) (layer "B.Cu") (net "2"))
 (segment (start 55.7 39.67) (end 51.495 39.67) (width 0.2) (layer "B.Cu") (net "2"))
 (segment (start 29.55 39.6) (end 26.675 42.475) (width 0.2) (layer "F.Cu") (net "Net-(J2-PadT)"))
 (segment (start 26.675 42.475) (end 26.675 43.05) (width 0.2) (layer "F.Cu") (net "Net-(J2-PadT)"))
 (segment (start 31.15 39.6) (end 29.55 39.6) (width 0.2) (layer "F.Cu") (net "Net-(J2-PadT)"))
 (segment (start 55.22 55.48) (end 53.98 54.24) (width 0.2) (layer "F.Cu") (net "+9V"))
 (segment (start 53.98 43.45) (end 53.98 45.75) (width 0.2) (layer "F.Cu") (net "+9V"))
 (segment (start 53.98 54.24) (end 53.98 45.75) (width 0.2) (layer "F.Cu") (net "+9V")))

